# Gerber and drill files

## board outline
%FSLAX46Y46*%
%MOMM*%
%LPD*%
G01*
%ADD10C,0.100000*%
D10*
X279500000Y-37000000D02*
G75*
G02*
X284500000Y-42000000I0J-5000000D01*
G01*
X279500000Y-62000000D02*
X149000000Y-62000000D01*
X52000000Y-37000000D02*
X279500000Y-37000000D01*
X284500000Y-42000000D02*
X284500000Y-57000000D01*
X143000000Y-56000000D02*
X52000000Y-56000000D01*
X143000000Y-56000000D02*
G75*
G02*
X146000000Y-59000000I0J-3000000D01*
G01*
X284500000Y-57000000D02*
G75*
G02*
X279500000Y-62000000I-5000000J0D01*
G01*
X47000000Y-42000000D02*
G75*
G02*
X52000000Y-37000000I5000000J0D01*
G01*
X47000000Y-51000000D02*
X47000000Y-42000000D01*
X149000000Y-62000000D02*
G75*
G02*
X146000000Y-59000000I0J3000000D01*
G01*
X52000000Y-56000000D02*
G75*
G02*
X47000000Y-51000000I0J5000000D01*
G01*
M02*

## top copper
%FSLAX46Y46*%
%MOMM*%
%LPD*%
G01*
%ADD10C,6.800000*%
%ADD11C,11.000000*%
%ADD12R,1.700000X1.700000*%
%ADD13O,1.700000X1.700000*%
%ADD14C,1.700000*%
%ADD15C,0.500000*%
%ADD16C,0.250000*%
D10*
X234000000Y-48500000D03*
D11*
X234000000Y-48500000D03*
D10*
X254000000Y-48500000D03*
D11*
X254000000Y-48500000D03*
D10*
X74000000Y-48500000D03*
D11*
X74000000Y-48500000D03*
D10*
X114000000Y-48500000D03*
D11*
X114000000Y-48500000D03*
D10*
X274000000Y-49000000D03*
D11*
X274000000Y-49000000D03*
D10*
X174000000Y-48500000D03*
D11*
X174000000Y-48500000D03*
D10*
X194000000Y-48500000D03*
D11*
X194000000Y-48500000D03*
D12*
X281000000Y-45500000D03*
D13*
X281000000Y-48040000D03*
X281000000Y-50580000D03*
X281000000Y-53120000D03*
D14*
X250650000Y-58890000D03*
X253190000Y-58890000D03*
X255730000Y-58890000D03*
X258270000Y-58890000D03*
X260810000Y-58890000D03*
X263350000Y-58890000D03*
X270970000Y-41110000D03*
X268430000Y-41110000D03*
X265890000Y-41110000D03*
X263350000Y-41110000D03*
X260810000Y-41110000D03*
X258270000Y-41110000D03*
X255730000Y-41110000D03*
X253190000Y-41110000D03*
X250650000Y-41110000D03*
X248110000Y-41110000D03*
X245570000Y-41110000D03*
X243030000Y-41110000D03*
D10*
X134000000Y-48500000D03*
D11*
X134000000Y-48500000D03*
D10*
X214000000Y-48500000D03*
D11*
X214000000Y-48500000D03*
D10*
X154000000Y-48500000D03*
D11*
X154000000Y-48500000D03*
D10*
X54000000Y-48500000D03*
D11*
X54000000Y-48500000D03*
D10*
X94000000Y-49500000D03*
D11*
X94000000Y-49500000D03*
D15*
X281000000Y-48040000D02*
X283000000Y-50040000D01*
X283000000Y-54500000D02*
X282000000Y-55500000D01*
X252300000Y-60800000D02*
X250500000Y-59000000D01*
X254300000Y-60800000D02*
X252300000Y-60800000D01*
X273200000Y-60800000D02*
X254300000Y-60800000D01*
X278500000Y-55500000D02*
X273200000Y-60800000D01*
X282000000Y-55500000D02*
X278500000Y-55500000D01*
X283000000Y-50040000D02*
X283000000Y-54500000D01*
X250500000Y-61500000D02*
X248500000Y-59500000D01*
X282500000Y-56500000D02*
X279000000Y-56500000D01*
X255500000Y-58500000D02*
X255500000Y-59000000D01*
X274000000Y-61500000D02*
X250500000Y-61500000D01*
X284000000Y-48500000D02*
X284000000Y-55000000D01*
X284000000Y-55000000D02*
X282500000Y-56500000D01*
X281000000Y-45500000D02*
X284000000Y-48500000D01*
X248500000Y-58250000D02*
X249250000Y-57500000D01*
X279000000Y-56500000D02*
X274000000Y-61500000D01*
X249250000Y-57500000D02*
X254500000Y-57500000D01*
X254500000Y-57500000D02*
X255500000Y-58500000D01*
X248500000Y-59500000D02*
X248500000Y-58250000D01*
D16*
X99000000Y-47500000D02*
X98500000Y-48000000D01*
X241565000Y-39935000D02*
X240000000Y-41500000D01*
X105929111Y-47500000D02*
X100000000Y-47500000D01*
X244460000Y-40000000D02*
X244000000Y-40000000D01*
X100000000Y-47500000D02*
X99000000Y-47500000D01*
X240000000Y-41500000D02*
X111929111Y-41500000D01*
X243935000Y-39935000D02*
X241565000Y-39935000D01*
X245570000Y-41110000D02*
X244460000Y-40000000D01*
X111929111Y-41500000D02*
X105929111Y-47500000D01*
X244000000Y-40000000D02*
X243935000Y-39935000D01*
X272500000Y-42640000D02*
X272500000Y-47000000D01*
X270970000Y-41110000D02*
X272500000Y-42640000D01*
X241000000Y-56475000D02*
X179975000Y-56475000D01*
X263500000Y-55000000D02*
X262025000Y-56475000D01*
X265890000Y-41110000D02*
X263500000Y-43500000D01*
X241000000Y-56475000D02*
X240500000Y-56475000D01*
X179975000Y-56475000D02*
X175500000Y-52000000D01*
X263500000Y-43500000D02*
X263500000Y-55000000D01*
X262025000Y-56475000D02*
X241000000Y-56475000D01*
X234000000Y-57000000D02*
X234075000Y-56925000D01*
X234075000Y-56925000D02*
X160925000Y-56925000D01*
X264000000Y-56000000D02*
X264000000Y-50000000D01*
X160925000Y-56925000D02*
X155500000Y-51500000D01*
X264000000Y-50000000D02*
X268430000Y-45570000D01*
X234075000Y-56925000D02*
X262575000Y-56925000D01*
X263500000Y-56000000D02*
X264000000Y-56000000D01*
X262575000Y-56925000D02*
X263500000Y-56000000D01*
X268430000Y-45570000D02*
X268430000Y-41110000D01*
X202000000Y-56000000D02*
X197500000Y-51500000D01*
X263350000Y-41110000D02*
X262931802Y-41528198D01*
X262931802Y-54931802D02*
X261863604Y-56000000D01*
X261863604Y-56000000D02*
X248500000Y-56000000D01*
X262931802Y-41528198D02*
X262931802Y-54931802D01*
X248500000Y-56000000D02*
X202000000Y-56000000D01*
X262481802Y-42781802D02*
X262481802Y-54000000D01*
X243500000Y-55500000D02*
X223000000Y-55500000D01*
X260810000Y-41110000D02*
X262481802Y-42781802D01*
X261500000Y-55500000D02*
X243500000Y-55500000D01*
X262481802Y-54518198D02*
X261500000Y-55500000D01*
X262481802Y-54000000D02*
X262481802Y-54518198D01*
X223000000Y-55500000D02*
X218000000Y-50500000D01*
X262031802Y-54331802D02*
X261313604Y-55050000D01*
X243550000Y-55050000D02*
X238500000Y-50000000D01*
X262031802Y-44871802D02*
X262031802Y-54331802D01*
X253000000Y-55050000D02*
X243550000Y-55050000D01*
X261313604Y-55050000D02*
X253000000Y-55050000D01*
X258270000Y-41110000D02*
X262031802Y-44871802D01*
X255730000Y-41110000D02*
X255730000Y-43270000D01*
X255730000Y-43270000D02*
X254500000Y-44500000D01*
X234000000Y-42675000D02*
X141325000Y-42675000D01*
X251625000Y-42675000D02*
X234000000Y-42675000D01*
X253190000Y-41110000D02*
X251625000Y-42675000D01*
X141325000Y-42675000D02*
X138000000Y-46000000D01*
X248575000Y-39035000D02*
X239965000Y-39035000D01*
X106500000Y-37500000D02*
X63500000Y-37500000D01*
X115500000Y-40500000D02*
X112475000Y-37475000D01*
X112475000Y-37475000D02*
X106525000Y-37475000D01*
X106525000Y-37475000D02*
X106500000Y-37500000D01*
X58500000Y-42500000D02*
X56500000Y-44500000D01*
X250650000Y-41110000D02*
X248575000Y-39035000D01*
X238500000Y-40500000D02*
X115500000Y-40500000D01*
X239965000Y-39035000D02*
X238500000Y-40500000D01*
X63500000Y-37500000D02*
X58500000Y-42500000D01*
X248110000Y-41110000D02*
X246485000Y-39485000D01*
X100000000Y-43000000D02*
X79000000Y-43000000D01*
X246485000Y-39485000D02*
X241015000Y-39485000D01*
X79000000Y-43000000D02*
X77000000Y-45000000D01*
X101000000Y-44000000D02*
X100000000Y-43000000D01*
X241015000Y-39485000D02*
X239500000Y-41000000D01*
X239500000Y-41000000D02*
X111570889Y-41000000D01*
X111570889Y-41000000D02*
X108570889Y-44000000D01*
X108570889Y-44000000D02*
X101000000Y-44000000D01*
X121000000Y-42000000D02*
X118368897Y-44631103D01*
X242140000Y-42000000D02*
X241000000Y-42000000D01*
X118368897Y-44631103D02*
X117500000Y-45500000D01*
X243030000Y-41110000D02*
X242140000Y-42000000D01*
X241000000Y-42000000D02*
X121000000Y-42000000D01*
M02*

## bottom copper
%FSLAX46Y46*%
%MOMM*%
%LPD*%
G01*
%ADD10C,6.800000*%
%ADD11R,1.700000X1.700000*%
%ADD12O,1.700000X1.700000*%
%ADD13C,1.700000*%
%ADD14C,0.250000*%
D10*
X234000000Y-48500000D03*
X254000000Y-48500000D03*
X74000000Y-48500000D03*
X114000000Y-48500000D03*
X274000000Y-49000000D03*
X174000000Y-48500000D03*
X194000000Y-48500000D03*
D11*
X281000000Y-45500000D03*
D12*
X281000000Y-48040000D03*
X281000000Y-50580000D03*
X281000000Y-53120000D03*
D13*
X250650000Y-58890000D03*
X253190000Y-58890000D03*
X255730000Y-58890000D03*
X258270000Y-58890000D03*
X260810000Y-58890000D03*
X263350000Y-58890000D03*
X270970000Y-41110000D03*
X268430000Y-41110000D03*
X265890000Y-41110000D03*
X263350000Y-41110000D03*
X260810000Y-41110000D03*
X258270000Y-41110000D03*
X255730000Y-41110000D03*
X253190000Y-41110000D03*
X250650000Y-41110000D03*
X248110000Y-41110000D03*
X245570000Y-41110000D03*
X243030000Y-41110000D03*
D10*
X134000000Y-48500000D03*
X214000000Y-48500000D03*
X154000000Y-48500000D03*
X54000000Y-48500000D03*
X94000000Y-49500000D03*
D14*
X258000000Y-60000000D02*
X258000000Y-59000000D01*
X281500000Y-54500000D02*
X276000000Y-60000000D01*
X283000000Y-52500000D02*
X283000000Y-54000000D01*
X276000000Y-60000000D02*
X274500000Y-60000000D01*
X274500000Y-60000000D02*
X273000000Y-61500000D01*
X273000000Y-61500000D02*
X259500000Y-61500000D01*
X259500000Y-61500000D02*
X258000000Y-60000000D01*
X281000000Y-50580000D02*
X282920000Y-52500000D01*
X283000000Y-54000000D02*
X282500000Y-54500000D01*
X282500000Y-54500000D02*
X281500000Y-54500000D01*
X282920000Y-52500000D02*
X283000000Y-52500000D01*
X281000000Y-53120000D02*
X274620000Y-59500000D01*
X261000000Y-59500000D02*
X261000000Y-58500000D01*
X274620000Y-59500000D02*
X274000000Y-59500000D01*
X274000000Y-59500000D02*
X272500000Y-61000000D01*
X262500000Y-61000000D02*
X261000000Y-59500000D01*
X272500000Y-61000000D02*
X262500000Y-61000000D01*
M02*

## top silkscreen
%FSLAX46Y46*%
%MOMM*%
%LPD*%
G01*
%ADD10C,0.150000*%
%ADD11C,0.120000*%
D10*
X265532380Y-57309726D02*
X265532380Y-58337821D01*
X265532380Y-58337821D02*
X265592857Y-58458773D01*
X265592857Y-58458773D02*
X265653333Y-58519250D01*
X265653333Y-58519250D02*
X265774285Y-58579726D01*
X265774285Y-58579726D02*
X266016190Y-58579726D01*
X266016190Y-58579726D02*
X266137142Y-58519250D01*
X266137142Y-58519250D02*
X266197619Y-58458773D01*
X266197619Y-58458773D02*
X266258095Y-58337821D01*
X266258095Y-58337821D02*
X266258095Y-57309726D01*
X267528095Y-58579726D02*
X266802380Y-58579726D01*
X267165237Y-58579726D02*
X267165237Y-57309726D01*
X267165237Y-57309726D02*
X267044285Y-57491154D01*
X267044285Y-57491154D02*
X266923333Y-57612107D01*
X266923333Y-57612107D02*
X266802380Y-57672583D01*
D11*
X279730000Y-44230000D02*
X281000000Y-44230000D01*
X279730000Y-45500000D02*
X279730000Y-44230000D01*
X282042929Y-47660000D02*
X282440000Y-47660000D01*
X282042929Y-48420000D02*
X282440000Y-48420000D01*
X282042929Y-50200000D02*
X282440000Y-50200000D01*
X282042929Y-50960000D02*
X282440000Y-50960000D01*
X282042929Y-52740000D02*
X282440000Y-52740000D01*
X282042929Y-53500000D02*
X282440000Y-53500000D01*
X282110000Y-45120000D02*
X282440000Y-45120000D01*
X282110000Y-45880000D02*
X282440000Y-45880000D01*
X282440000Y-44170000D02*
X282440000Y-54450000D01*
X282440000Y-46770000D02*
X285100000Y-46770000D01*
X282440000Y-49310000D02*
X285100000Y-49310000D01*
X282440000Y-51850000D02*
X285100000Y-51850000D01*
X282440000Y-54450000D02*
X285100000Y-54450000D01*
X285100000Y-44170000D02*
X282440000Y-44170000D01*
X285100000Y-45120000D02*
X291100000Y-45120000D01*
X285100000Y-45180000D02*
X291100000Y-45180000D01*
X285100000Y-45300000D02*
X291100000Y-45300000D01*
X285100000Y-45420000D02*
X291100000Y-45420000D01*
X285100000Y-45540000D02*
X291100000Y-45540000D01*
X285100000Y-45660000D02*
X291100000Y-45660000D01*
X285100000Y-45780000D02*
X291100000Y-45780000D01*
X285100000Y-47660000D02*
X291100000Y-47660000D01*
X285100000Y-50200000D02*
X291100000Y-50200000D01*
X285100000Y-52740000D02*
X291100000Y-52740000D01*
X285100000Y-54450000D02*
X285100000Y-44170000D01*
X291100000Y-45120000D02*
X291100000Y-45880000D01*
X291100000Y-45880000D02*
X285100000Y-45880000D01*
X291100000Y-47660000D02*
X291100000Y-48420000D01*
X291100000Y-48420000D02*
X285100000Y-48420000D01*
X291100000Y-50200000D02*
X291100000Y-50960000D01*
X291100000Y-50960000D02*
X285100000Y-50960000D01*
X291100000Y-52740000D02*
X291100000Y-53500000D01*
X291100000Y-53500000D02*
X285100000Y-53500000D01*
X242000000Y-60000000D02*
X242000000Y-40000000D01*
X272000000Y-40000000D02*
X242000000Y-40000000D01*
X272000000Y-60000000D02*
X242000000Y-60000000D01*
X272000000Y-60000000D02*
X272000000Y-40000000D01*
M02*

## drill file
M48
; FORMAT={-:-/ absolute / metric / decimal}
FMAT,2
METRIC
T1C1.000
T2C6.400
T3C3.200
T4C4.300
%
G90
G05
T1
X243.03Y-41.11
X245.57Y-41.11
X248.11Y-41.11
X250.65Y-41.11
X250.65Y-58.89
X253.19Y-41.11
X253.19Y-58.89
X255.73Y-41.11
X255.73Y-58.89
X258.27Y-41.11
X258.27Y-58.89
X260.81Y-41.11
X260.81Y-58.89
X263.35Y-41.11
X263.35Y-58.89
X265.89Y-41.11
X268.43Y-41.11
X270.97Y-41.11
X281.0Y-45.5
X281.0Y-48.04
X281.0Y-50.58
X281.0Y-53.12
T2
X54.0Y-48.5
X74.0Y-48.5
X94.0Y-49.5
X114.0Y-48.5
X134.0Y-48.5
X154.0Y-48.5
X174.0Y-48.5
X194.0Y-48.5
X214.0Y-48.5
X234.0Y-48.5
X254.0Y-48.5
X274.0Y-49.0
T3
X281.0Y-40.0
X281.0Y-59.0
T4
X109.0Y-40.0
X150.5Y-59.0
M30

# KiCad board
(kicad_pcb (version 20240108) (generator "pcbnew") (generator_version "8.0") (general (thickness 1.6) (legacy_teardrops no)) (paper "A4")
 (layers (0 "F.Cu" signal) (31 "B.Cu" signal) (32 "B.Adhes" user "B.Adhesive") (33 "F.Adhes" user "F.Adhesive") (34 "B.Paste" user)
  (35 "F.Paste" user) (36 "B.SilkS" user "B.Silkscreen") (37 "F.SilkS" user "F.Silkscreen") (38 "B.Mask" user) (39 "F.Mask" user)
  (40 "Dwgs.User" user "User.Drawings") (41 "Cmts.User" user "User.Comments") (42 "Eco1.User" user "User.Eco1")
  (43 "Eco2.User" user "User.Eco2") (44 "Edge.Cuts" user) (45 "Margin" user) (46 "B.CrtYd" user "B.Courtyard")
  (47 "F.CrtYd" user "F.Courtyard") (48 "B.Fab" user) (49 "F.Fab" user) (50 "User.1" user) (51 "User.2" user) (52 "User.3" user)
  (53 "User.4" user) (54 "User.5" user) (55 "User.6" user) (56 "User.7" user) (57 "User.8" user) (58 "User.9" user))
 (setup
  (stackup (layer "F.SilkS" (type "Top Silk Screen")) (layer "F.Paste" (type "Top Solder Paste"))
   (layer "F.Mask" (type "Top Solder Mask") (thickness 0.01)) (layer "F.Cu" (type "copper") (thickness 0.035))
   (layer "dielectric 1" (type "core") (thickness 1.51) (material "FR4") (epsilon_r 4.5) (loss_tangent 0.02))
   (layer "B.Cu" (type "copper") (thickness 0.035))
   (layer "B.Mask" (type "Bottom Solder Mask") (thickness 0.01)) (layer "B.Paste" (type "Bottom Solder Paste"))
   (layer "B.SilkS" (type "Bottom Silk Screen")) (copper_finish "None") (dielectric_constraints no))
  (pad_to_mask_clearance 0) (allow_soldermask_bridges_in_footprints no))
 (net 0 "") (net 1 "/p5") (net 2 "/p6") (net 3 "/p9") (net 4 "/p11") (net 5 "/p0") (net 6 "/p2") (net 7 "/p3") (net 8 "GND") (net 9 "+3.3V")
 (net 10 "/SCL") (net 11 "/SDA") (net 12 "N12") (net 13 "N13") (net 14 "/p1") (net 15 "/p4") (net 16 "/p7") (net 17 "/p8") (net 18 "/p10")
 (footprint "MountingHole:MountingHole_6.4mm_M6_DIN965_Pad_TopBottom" (layer "F.Cu") (at 234 48.5 90)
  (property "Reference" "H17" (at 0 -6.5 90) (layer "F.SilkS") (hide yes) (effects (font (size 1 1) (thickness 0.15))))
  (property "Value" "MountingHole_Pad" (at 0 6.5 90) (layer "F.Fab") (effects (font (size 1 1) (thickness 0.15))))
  (pad "" connect circle (at 0 0 90) (size 11 11) (layers "B.Mask" "Rescue"))
  (pad "1" thru_hole circle (at 0 0 90) (size 6.8 6.8) (drill 6.4) (layers "*.Cu" "*.Mask") (remove_unused_layers no) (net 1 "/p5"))
  (pad "1" connect circle (at 0 0 90) (size 11 11) (layers "F.Cu" "F.Mask") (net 1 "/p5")))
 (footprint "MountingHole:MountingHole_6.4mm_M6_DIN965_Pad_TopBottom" (layer "F.Cu") (at 254 48.5 90)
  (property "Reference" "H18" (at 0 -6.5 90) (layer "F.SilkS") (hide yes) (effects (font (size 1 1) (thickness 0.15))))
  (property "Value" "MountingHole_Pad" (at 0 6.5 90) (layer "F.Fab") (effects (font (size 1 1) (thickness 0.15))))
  (pad "" connect circle (at 0 0 90) (size 11 11) (layers "B.Mask" "Rescue"))
  (pad "1" thru_hole circle (at 0 0 90) (size 6.8 6.8) (drill 6.4) (layers "*.Cu" "*.Mask") (remove_unused_layers no) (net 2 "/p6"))
  (pad "1" connect circle (at 0 0 90) (size 11 11) (layers "F.Cu" "F.Mask") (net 2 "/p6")))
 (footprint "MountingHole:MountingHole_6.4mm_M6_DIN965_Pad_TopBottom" (layer "F.Cu") (at 74 48.5)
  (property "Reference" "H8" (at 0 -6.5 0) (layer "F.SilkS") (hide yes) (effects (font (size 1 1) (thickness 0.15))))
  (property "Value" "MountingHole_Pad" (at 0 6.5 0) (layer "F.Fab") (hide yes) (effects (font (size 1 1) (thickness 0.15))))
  (pad "" connect circle (at 0 0) (size 11 11) (layers "B.Mask" "Rescue"))
  (pad "1" thru_hole circle (at 0 0) (size 6.8 6.8) (drill 6.4) (layers "*.Cu" "*.Mask") (remove_unused_layers no) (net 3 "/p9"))
  (pad "1" connect circle (at 0 0) (size 11 11) (layers "F.Cu" "F.Mask") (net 3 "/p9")))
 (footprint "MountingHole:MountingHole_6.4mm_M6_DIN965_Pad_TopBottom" (layer "F.Cu") (at 114 48.5 90)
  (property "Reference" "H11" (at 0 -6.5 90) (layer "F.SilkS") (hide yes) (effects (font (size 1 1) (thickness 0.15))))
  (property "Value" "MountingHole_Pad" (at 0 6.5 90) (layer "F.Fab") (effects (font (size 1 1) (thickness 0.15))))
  (pad "" connect circle (at 0 0 90) (size 11 11) (layers "B.Mask" "Rescue"))
  (pad "1" thru_hole circle (at 0 0 90) (size 6.8 6.8) (drill 6.4) (layers "*.Cu" "*.Mask") (remove_unused_layers no) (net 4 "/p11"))
  (pad "1" connect circle (at 0 0 90) (size 11 11) (layers "F.Cu" "F.Mask") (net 4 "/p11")))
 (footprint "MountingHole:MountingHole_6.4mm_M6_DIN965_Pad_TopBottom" (layer "F.Cu") (at 274 49 90)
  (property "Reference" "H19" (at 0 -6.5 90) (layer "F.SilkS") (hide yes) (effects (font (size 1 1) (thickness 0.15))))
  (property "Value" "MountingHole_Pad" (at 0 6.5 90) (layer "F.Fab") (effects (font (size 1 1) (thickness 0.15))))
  (pad "" connect circle (at 0 0 90) (size 11 11) (layers "B.Mask" "Rescue"))
  (pad "1" thru_hole circle (at 0 0 90) (size 6.8 6.8) (drill 6.4) (layers "*.Cu" "*.Mask") (remove_unused_layers no) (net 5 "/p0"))
  (pad "1" connect circle (at 0 0 90) (size 11 11) (layers "F.Cu" "F.Mask") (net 5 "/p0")))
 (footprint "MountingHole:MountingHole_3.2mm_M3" (layer "F.Cu") (at 283.7475 40.08 -90)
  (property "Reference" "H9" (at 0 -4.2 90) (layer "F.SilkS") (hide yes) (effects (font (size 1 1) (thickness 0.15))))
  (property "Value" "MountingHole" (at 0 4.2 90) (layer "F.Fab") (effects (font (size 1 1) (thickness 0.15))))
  (pad "" np_thru_hole circle (at -0.08 2.7475 270) (size 3.2 3.2) (drill 3.2) (layers "F&B.Cu" "*.Mask")))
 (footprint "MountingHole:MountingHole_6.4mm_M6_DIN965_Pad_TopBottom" (layer "F.Cu") (at 174 48.5 90)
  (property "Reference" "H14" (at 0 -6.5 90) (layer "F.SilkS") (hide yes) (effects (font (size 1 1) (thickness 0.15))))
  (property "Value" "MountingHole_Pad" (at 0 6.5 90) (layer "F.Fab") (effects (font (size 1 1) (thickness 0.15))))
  (pad "" connect circle (at 0 0 90) (size 11 11) (layers "B.Mask" "Rescue"))
  (pad "1" thru_hole circle (at 0 0 90) (size 6.8 6.8) (drill 6.4) (layers "*.Cu" "*.Mask") (remove_unused_layers no) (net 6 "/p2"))
  (pad "1" connect circle (at 0 0 90) (size 11 11) (layers "F.Cu" "F.Mask") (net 6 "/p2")))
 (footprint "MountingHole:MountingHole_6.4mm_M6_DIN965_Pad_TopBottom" (layer "F.Cu") (at 194 48.5 90)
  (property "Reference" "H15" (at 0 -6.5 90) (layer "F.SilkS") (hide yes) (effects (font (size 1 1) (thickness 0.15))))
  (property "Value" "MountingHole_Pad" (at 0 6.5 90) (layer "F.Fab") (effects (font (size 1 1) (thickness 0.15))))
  (pad "" connect circle (at 0 0 90) (size 11 11) (layers "B.Mask" "Rescue"))
  (pad "1" thru_hole circle (at 0 0 90) (size 6.8 6.8) (drill 6.4) (layers "*.Cu" "*.Mask") (remove_unused_layers no) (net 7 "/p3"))
  (pad "1" connect circle (at 0 0 90) (size 11 11) (layers "F.Cu" "F.Mask") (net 7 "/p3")))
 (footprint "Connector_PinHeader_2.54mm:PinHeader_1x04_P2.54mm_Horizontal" (layer "F.Cu") (at 281 45.5)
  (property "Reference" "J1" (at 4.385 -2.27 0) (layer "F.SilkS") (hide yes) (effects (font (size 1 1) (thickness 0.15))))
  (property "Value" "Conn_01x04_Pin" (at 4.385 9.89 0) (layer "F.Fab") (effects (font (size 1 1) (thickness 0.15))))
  (fp_line (start -1.27 -1.27) (end 0 -1.27) (stroke (width 0.12) (type solid)) (layer "F.SilkS"))
  (fp_line (start -1.27 0) (end -1.27 -1.27) (stroke (width 0.12) (type solid)) (layer "F.SilkS"))
  (fp_line (start 1.042929 2.16) (end 1.44 2.16) (stroke (width 0.12) (type solid)) (layer "F.SilkS"))
  (fp_line (start 1.042929 2.92) (end 1.44 2.92) (stroke (width 0.12) (type solid)) (layer "F.SilkS"))
  (fp_line (start 1.042929 4.7) (end 1.44 4.7) (stroke (width 0.12) (type solid)) (layer "F.SilkS"))
  (fp_line (start 1.042929 5.46) (end 1.44 5.46) (stroke (width 0.12) (type solid)) (layer "F.SilkS"))
  (fp_line (start 1.042929 7.24) (end 1.44 7.24) (stroke (width 0.12) (type solid)) (layer "F.SilkS"))
  (fp_line (start 1.042929 8) (end 1.44 8) (stroke (width 0.12) (type solid)) (layer "F.SilkS"))
  (fp_line (start 1.11 -0.38) (end 1.44 -0.38) (stroke (width 0.12) (type solid)) (layer "F.SilkS"))
  (fp_line (start 1.11 0.38) (end 1.44 0.38) (stroke (width 0.12) (type solid)) (layer "F.SilkS"))
  (fp_line (start 1.44 -1.33) (end 1.44 8.95) (stroke (width 0.12) (type solid)) (layer "F.SilkS"))
  (fp_line (start 1.44 1.27) (end 4.1 1.27) (stroke (width 0.12) (type solid)) (layer "F.SilkS"))
  (fp_line (start 1.44 3.81) (end 4.1 3.81) (stroke (width 0.12) (type solid)) (layer "F.SilkS"))
  (fp_line (start 1.44 6.35) (end 4.1 6.35) (stroke (width 0.12) (type solid)) (layer "F.SilkS"))
  (fp_line (start 1.44 8.95) (end 4.1 8.95) (stroke (width 0.12) (type solid)) (layer "F.SilkS"))
  (fp_line (start 4.1 -1.33) (end 1.44 -1.33) (stroke (width 0.12) (type solid)) (layer "F.SilkS"))
  (fp_line (start 4.1 -0.38) (end 10.1 -0.38) (stroke (width 0.12) (type solid)) (layer "F.SilkS"))
  (fp_line (start 4.1 -0.32) (end 10.1 -0.32) (stroke (width 0.12) (type solid)) (layer "F.SilkS"))
  (fp_line (start 4.1 -0.2) (end 10.1 -0.2) (stroke (width 0.12) (type solid)) (layer "F.SilkS"))
  (fp_line (start 4.1 -0.08) (end 10.1 -0.08) (stroke (width 0.12) (type solid)) (layer "F.SilkS"))
  (fp_line (start 4.1 0.04) (end 10.1 0.04) (stroke (width 0.12) (type solid)) (layer "F.SilkS"))
  (fp_line (start 4.1 0.16) (end 10.1 0.16) (stroke (width 0.12) (type solid)) (layer "F.SilkS"))
  (fp_line (start 4.1 0.28) (end 10.1 0.28) (stroke (width 0.12) (type solid)) (layer "F.SilkS"))
  (fp_line (start 4.1 2.16) (end 10.1 2.16) (stroke (width 0.12) (type solid)) (layer "F.SilkS"))
  (fp_line (start 4.1 4.7) (end 10.1 4.7) (stroke (width 0.12) (type solid)) (layer "F.SilkS"))
  (fp_line (start 4.1 7.24) (end 10.1 7.24) (stroke (width 0.12) (type solid)) (layer "F.SilkS"))
  (fp_line (start 4.1 8.95) (end 4.1 -1.33) (stroke (width 0.12) (type solid)) (layer "F.SilkS"))
  (fp_line (start 10.1 -0.38) (end 10.1 0.38) (stroke (width 0.12) (type solid)) (layer "F.SilkS"))
  (fp_line (start 10.1 0.38) (end 4.1 0.38) (stroke (width 0.12) (type solid)) (layer "F.SilkS"))
  (fp_line (start 10.1 2.16) (end 10.1 2.92) (stroke (width 0.12) (type solid)) (layer "F.SilkS"))
  (fp_line (start 10.1 2.92) (end 4.1 2.92) (stroke (width 0.12) (type solid)) (layer "F.SilkS"))
  (fp_line (start 10.1 4.7) (end 10.1 5.46) (stroke (width 0.12) (type solid)) (layer "F.SilkS"))
  (fp_line (start 10.1 5.46) (end 4.1 5.46) (stroke (width 0.12) (type solid)) (layer "F.SilkS"))
  (fp_line (start 10.1 7.24) (end 10.1 8) (stroke (width 0.12) (type solid)) (layer "F.SilkS"))
  (fp_line (start 10.1 8) (end 4.1 8) (stroke (width 0.12) (type solid)) (layer "F.SilkS"))
  (pad "1" thru_hole rect (at 0 0) (size 1.7 1.7) (drill 1) (layers "*.Cu" "*.Mask") (remove_unused_layers no) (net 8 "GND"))
  (pad "2" thru_hole oval (at 0 2.54) (size 1.7 1.7) (drill 1) (layers "*.Cu" "*.Mask") (remove_unused_layers no) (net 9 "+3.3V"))
  (pad "3" thru_hole oval (at 0 5.08) (size 1.7 1.7) (drill 1) (layers "*.Cu" "*.Mask") (remove_unused_layers no) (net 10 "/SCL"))
  (pad "4" thru_hole oval (at 0 7.62) (size 1.7 1.7) (drill 1) (layers "*.Cu" "*.Mask") (remove_unused_layers no) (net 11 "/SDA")))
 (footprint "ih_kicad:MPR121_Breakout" (layer "F.Cu") (at 257 50 180)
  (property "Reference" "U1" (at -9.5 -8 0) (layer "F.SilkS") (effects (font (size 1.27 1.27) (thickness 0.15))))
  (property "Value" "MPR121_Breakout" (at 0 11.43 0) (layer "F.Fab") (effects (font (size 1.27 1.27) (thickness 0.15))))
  (fp_line (start 15 -10) (end 15 10) (stroke (width 0.12) (type solid)) (layer "F.SilkS"))
  (fp_line (start -15 10) (end 15 10) (stroke (width 0.12) (type solid)) (layer "F.SilkS"))
  (fp_line (start -15 -10) (end 15 -10) (stroke (width 0.12) (type solid)) (layer "F.SilkS"))
  (fp_line (start -15 -10) (end -15 10) (stroke (width 0.12) (type solid)) (layer "F.SilkS"))
  (pad "1" thru_hole circle (at 6.35 -8.89 180) (size 1.7 1.7) (drill 1) (layers "*.Cu" "*.Mask") (remove_unused_layers no) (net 9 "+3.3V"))
  (pad "2" thru_hole circle (at 3.81 -8.89 180) (size 1.7 1.7) (drill 1) (layers "*.Cu" "*.Mask") (remove_unused_layers no) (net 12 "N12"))
  (pad "3" thru_hole circle (at 1.27 -8.89 180) (size 1.7 1.7) (drill 1) (layers "*.Cu" "*.Mask") (remove_unused_layers no) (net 8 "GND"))
  (pad "4" thru_hole circle (at -1.27 -8.89 180) (size 1.7 1.7) (drill 1) (layers "*.Cu" "*.Mask") (remove_unused_layers no) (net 10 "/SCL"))
  (pad "5" thru_hole circle (at -3.81 -8.89 180) (size 1.7 1.7) (drill 1) (layers "*.Cu" "*.Mask") (remove_unused_layers no) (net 11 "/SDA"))
  (pad "6" thru_hole circle (at -6.35 -8.89 180) (size 1.7 1.7) (drill 1) (layers "*.Cu" "*.Mask") (remove_unused_layers no) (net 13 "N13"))
  (pad "7" thru_hole circle (at -13.97 8.89 180) (size 1.7 1.7) (drill 1) (layers "*.Cu" "*.Mask") (remove_unused_layers no) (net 5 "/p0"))
  (pad "8" thru_hole circle (at -11.43 8.89 180) (size 1.7 1.7) (drill 1) (layers "*.Cu" "*.Mask") (remove_unused_layers no) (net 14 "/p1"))
  (pad "9" thru_hole circle (at -8.89 8.89 180) (size 1.7 1.7) (drill 1) (layers "*.Cu" "*.Mask") (remove_unused_layers no) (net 6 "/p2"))
  (pad "10" thru_hole circle (at -6.35 8.89 180) (size 1.7 1.7) (drill 1) (layers "*.Cu" "*.Mask") (remove_unused_layers no) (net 7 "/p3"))
  (pad "11" thru_hole circle (at -3.81 8.89 180) (size 1.7 1.7) (drill 1) (layers "*.Cu" "*.Mask") (remove_unused_layers no) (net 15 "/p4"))
  (pad "12" thru_hole circle (at -1.27 8.89 180) (size 1.7 1.7) (drill 1) (layers "*.Cu" "*.Mask") (remove_unused_layers no) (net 1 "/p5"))
  (pad "13" thru_hole circle (at 1.27 8.89 180) (size 1.7 1.7) (drill 1) (layers "*.Cu" "*.Mask") (remove_unused_layers no) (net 2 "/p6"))
  (pad "14" thru_hole circle (at 3.81 8.89 180) (size 1.7 1.7) (drill 1) (layers "*.Cu" "*.Mask") (remove_unused_layers no) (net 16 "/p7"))
  (pad "15" thru_hole circle (at 6.35 8.89 180) (size 1.7 1.7) (drill 1) (layers "*.Cu" "*.Mask") (remove_unused_layers no) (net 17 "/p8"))
  (pad "16" thru_hole circle (at 8.89 8.89 180) (size 1.7 1.7) (drill 1) (layers "*.Cu" "*.Mask") (remove_unused_layers no) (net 3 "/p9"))
  (pad "17" thru_hole circle (at 11.43 8.89 180) (size 1.7 1.7) (drill 1) (layers "*.Cu" "*.Mask") (remove_unused_layers no) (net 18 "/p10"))
  (pad "18" thru_hole circle (at 13.97 8.89 180) (size 1.7 1.7) (drill 1) (layers "*.Cu" "*.Mask") (remove_unused_layers no) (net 4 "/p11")))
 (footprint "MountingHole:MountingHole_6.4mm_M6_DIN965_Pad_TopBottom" (layer "F.Cu") (at 134 48.5 90)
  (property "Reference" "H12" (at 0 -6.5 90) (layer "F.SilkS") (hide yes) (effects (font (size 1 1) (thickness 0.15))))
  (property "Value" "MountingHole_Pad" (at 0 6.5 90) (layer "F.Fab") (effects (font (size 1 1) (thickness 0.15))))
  (pad "" connect circle (at 0 0 90) (size 11 11) (layers "B.Mask" "Rescue"))
  (pad "1" thru_hole circle (at 0 0 90) (size 6.8 6.8) (drill 6.4) (layers "*.Cu" "*.Mask") (remove_unused_layers no) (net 16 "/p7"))
  (pad "1" connect circle (at 0 0 90) (size 11 11) (layers "F.Cu" "F.Mask") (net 16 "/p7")))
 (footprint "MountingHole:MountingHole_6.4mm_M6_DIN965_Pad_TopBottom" (layer "F.Cu") (at 214 48.5 90)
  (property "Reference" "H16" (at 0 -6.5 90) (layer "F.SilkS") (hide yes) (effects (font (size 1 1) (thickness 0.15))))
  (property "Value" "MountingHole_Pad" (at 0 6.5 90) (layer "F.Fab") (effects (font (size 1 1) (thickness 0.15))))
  (pad "" connect circle (at 0 0 90) (size 11 11) (layers "B.Mask" "Rescue"))
  (pad "1" thru_hole circle (at 0 0 90) (size 6.8 6.8) (drill 6.4) (layers "*.Cu" "*.Mask") (remove_unused_layers no) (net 15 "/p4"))
  (pad "1" connect circle (at 0 0 90) (size 11 11) (layers "F.Cu" "F.Mask") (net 15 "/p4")))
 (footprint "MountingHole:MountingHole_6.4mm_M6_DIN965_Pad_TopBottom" (layer "F.Cu") (at 154 48.5 90)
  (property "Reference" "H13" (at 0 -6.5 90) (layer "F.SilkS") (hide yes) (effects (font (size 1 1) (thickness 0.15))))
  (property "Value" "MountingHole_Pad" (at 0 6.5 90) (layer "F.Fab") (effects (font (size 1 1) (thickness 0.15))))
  (pad "" connect circle (at 0 0 90) (size 11 11) (layers "B.Mask" "Rescue"))
  (pad "1" thru_hole circle (at 0 0 90) (size 6.8 6.8) (drill 6.4) (layers "*.Cu" "*.Mask") (remove_unused_layers no) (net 14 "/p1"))
  (pad "1" connect circle (at 0 0 90) (size 11 11) (layers "F.Cu" "F.Mask") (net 14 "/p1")))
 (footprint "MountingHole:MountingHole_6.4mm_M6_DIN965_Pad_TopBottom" (layer "F.Cu") (at 54 48.5)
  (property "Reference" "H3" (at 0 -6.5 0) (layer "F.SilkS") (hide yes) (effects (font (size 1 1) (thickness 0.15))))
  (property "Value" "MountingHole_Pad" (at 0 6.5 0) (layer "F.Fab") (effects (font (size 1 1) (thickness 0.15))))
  (pad "" connect circle (at 0 0) (size 11 11) (layers "B.Mask" "Rescue"))
  (pad "1" thru_hole circle (at 0 0) (size 6.8 6.8) (drill 6.4) (layers "*.Cu" "*.Mask") (remove_unused_layers no) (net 17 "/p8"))
  (pad "1" connect circle (at 0 0) (size 11 11) (layers "F.Cu" "F.Mask") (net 17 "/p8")))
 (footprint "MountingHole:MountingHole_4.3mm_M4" (layer "F.Cu") (at 118 97.5)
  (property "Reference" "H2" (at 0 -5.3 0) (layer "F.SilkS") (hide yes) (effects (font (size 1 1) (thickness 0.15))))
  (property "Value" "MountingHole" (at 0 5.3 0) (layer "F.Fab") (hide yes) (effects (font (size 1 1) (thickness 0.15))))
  (pad "" np_thru_hole circle (at -9 -57.5) (size 4.3 4.3) (drill 4.3) (layers "F&B.Cu" "*.Mask")))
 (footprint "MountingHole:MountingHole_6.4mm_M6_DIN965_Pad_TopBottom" (layer "F.Cu") (at 94 49.5)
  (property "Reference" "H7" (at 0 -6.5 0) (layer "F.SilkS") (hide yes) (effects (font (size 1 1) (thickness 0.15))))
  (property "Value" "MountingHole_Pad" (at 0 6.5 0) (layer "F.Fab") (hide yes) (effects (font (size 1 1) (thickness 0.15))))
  (pad "" connect circle (at 0 0) (size 11 11) (layers "B.Mask" "Rescue"))
  (pad "1" thru_hole circle (at 0 0) (size 6.8 6.8) (drill 6.4) (layers "*.Cu" "*.Mask") (remove_unused_layers no) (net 18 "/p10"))
  (pad "1" connect circle (at 0 0) (size 11 11) (layers "F.Cu" "F.Mask") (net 18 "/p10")))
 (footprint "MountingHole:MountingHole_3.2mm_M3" (layer "F.Cu") (at 278.7475 74.58 -90)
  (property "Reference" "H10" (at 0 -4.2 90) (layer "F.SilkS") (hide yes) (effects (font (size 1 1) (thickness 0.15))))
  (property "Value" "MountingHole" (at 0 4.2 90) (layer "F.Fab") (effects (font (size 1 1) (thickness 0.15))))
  (pad "" np_thru_hole circle (at -15.58 -2.2525 270) (size 3.2 3.2) (drill 3.2) (layers "F&B.Cu" "*.Mask")))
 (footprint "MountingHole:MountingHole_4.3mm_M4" (layer "F.Cu") (at 146.5 97.5)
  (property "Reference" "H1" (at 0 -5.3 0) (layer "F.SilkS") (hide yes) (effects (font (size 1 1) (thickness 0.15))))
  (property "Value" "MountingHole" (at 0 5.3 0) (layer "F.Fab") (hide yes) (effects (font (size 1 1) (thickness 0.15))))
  (pad "" np_thru_hole circle (at 4 -38.5) (size 4.3 4.3) (drill 4.3) (layers "F&B.Cu" "*.Mask")))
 (gr_arc (start 279.5 37) (mid 283.035534 38.464466) (end 284.5 42) (stroke (width 0.1) (type default)) (layer "Edge.Cuts"))
 (gr_line (start 279.5 62) (end 149 62) (stroke (width 0.1) (type default)) (layer "Edge.Cuts"))
 (gr_line (start 52 37) (end 279.5 37) (stroke (width 0.1) (type default)) (layer "Edge.Cuts"))
 (gr_line (start 284.5 42) (end 284.5 57) (stroke (width 0.1) (type default)) (layer "Edge.Cuts"))
 (gr_line (start 143 56) (end 52 56) (stroke (width 0.1) (type default)) (layer "Edge.Cuts"))
 (gr_arc (start 143 56) (mid 145.12132 56.87868) (end 146 59) (stroke (width 0.1) (type default)) (layer "Edge.Cuts"))
 (gr_arc (start 284.5 57) (mid 283.035534 60.535534) (end 279.5 62) (stroke (width 0.1) (type default)) (layer "Edge.Cuts"))
 (gr_arc (start 47 42) (mid 48.464466 38.464466) (end 52 37) (stroke (width 0.1) (type default)) (layer "Edge.Cuts"))
 (gr_line (start 47 51) (end 47 42) (stroke (width 0.1) (type default)) (layer "Edge.Cuts"))
 (gr_arc (start 149 62) (mid 146.87868 61.12132) (end 146 59) (stroke (width 0.1) (type default)) (layer "Edge.Cuts"))
 (gr_arc (start 52 56) (mid 48.464466 54.535534) (end 47 51) (stroke (width 0.1) (type default)) (layer "Edge.Cuts"))
 (segment (start 281 48.04) (end 283 50.04) (width 0.5) (layer "F.Cu") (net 9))
 (segment (start 283 54.5) (end 282 55.5) (width 0.5) (layer "F.Cu") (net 9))
 (segment (start 252.3 60.8) (end 250.5 59) (width 0.5) (layer "F.Cu") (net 9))
 (segment (start 254.3 60.8) (end 252.3 60.8) (width 0.5) (layer "F.Cu") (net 9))
 (segment (start 273.2 60.8) (end 254.3 60.8) (width 0.5) (layer "F.Cu") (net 9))
 (segment (start 278.5 55.5) (end 273.2 60.8) (width 0.5) (layer "F.Cu") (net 9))
 (segment (start 282 55.5) (end 278.5 55.5) (width 0.5) (layer "F.Cu") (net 9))
 (segment (start 283 50.04) (end 283 54.5) (width 0.5) (layer "F.Cu") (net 9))
 (segment (start 250.5 61.5) (end 248.5 59.5) (width 0.5) (layer "F.Cu") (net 8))
 (segment (start 282.5 56.5) (end 279 56.5) (width 0.5) (layer "F.Cu") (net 8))
 (segment (start 255.5 58.5) (end 255.5 59) (width 0.5) (layer "F.Cu") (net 8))
 (segment (start 274 61.5) (end 250.5 61.5) (width 0.5) (layer "F.Cu") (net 8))
 (segment (start 284 48.5) (end 284 55) (width 0.5) (layer "F.Cu") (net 8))
 (segment (start 284 55) (end 282.5 56.5) (width 0.5) (layer "F.Cu") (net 8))
 (segment (start 281 45.5) (end 284 48.5) (width 0.5) (layer "F.Cu") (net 8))
 (segment (start 248.5 58.25) (end 249.25 57.5) (width 0.5) (layer "F.Cu") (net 8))
 (segment (start 279 56.5) (end 274 61.5) (width 0.5) (layer "F.Cu") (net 8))
 (segment (start 249.25 57.5) (end 254.5 57.5) (width 0.5) (layer "F.Cu") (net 8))
 (segment (start 254.5 57.5) (end 255.5 58.5) (width 0.5) (layer "F.Cu") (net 8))
 (segment (start 248.5 59.5) (end 248.5 58.25) (width 0.5) (layer "F.Cu") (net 8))
 (segment (start 99 47.5) (end 98.5 48) (width 0.25) (layer "F.Cu") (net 18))
 (segment (start 241.565 39.935) (end 240 41.5) (width 0.25) (layer "F.Cu") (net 18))
 (segment (start 105.929111 47.5) (end 100 47.5) (width 0.25) (layer "F.Cu") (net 18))
 (segment (start 244.46 40) (end 244 40) (width 0.25) (layer "F.Cu") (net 18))
 (segment (start 100 47.5) (end 99 47.5) (width 0.25) (layer "F.Cu") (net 18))
 (segment (start 240 41.5) (end 111.929111 41.5) (width 0.25) (layer "F.Cu") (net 18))
 (segment (start 243.935 39.935) (end 241.565 39.935) (width 0.25) (layer "F.Cu") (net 18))
 (segment (start 245.57 41.11) (end 244.46 40) (width 0.25) (layer "F.Cu") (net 18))
 (segment (start 111.929111 41.5) (end 105.929111 47.5) (width 0.25) (layer "F.Cu") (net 18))
 (segment (start 244 40) (end 243.935 39.935) (width 0.25) (layer "F.Cu") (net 18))
 (segment (start 272.5 42.64) (end 272.5 47) (width 0.25) (layer "F.Cu") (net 5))
 (segment (start 270.97 41.11) (end 272.5 42.64) (width 0.25) (layer "F.Cu") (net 5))
 (segment (start 241 56.475) (end 179.975 56.475) (width 0.25) (layer "F.Cu") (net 6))
 (segment (start 263.5 55) (end 262.025 56.475) (width 0.25) (layer "F.Cu") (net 6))
 (segment (start 265.89 41.11) (end 263.5 43.5) (width 0.25) (layer "F.Cu") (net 6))
 (segment (start 241 56.475) (end 240.5 56.475) (width 0.25) (layer "F.Cu") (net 6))
 (segment (start 179.975 56.475) (end 175.5 52) (width 0.25) (layer "F.Cu") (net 6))
 (segment (start 263.5 43.5) (end 263.5 55) (width 0.25) (layer "F.Cu") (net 6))
 (segment (start 262.025 56.475) (end 241 56.475) (width 0.25) (layer "F.Cu") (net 6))
 (segment (start 258 60) (end 258 59) (width 0.25) (layer "B.Cu") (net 10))
 (segment (start 281.5 54.5) (end 276 60) (width 0.25) (layer "B.Cu") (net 10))
 (segment (start 283 52.5) (end 283 54) (width 0.25) (layer "B.Cu") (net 10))
 (segment (start 276 60) (end 274.5 60) (width 0.25) (layer "B.Cu") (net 10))
 (segment (start 274.5 60) (end 273 61.5) (width 0.25) (layer "B.Cu") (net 10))
 (segment (start 273 61.5) (end 259.5 61.5) (width 0.25) (layer "B.Cu") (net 10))
 (segment (start 259.5 61.5) (end 258 60) (width 0.25) (layer "B.Cu") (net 10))
 (segment (start 281 50.58) (end 282.92 52.5) (width 0.25) (layer "B.Cu") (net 10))
 (segment (start 283 54) (end 282.5 54.5) (width 0.25) (layer "B.Cu") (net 10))
 (segment (start 282.5 54.5) (end 281.5 54.5) (width 0.25) (layer "B.Cu") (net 10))
 (segment (start 282.92 52.5) (end 283 52.5) (width 0.25) (layer "B.Cu") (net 10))
 (segment (start 281 53.12) (end 274.62 59.5) (width 0.25) (layer "B.Cu") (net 11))
 (segment (start 261 59.5) (end 261 58.5) (width 0.25) (layer "B.Cu") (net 11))
 (segment (start 274.62 59.5) (end 274 59.5) (width 0.25) (layer "B.Cu") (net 11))
 (segment (start 274 59.5) (end 272.5 61) (width 0.25) (layer "B.Cu") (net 11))
 (segment (start 262.5 61) (end 261 59.5) (width 0.25) (layer "B.Cu") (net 11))
 (segment (start 272.5 61) (end 262.5 61) (width 0.25) (layer "B.Cu") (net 11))
 (segment (start 234 57) (end 234.075 56.925) (width 0.25) (layer "F.Cu") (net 14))
 (segment (start 234.075 56.925) (end 160.925 56.925) (width 0.25) (layer "F.Cu") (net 14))
 (segment (start 264 56) (end 264 50) (width 0.25) (layer "F.Cu") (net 14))
 (segment (start 160.925 56.925) (end 155.5 51.5) (width 0.25) (layer "F.Cu") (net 14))
 (segment (start 264 50) (end 268.43 45.57) (width 0.25) (layer "F.Cu") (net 14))
 (segment (start 234.075 56.925) (end 262.575 56.925) (width 0.25) (layer "F.Cu") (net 14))
 (segment (start 263.5 56) (end 264 56) (width 0.25) (layer "F.Cu") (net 14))
 (segment (start 262.575 56.925) (end 263.5 56) (width 0.25) (layer "F.Cu") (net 14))
 (segment (start 268.43 45.57) (end 268.43 41.11) (width 0.25) (layer "F.Cu") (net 14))
 (segment (start 202 56) (end 197.5 51.5) (width 0.25) (layer "F.Cu") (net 7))
 (segment (start 263.35 41.11) (end 262.931802 41.528198) (width 0.25) (layer "F.Cu") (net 7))
 (segment (start 262.931802 54.931802) (end 261.863604 56) (width 0.25) (layer "F.Cu") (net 7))
 (segment (start 261.863604 56) (end 248.5 56) (width 0.25) (layer "F.Cu") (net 7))
 (segment (start 262.931802 41.528198) (end 262.931802 54.931802) (width 0.25) (layer "F.Cu") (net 7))
 (segment (start 248.5 56) (end 202 56) (width 0.25) (layer "F.Cu") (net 7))
 (segment (start 262.481802 42.781802) (end 262.481802 54) (width 0.25) (layer "F.Cu") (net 15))
 (segment (start 243.5 55.5) (end 223 55.5) (width 0.25) (layer "F.Cu") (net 15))
 (segment (start 260.81 41.11) (end 262.481802 42.781802) (width 0.25) (layer "F.Cu") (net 15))
 (segment (start 261.5 55.5) (end 243.5 55.5) (width 0.25) (layer "F.Cu") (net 15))
 (segment (start 262.481802 54.518198) (end 261.5 55.5) (width 0.25) (layer "F.Cu") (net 15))
 (segment (start 262.481802 54) (end 262.481802 54.518198) (width 0.25) (layer "F.Cu") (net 15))
 (segment (start 223 55.5) (end 218 50.5) (width 0.25) (layer "F.Cu") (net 15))
 (segment (start 262.031802 54.331802) (end 261.313604 55.05) (width 0.25) (layer "F.Cu") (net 1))
 (segment (start 243.55 55.05) (end 238.5 50) (width 0.25) (layer "F.Cu") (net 1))
 (segment (start 262.031802 44.871802) (end 262.031802 54.331802) (width 0.25) (layer "F.Cu") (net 1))
 (segment (start 253 55.05) (end 243.55 55.05) (width 0.25) (layer "F.Cu") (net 1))
 (segment (start 261.313604 55.05) (end 253 55.05) (width 0.25) (layer "F.Cu") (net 1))
 (segment (start 258.27 41.11) (end 262.031802 44.871802) (width 0.25) (layer "F.Cu") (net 1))
 (segment (start 255.73 41.11) (end 255.73 43.27) (width 0.25) (layer "F.Cu") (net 2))
 (segment (start 255.73 43.27) (end 254.5 44.5) (width 0.25) (layer "F.Cu") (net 2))
 (segment (start 234 42.675) (end 141.325 42.675) (width 0.25) (layer "F.Cu") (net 16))
 (segment (start 251.625 42.675) (end 234 42.675) (width 0.25) (layer "F.Cu") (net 16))
 (segment (start 253.19 41.11) (end 251.625 42.675) (width 0.25) (layer "F.Cu") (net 16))
 (segment (start 141.325 42.675) (end 138 46) (width 0.25) (layer "F.Cu") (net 16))
 (segment (start 248.575 39.035) (end 239.965 39.035) (width 0.25) (layer "F.Cu") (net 17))
 (segment (start 106.5 37.5) (end 63.5 37.5) (width 0.25) (layer "F.Cu") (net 17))
 (segment (start 115.5 40.5) (end 112.475 37.475) (width 0.25) (layer "F.Cu") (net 17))
 (segment (start 112.475 37.475) (end 106.525 37.475) (width 0.25) (layer "F.Cu") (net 17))
 (segment (start 106.525 37.475) (end 106.5 37.5) (width 0.25) (layer "F.Cu") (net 17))
 (segment (start 58.5 42.5) (end 56.5 44.5) (width 0.25) (layer "F.Cu") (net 17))
 (segment (start 250.65 41.11) (end 248.575 39.035) (width 0.25) (layer "F.Cu") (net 17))
 (segment (start 238.5 40.5) (end 115.5 40.5) (width 0.25) (layer "F.Cu") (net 17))
 (segment (start 239.965 39.035) (end 238.5 40.5) (width 0.25) (layer "F.Cu") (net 17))
 (segment (start 63.5 37.5) (end 58.5 42.5) (width 0.25) (layer "F.Cu") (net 17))
 (segment (start 248.11 41.11) (end 246.485 39.485) (width 0.25) (layer "F.Cu") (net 3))
 (segment (start 100 43) (end 79 43) (width 0.25) (layer "F.Cu") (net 3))
 (segment (start 246.485 39.485) (end 241.015 39.485) (width 0.25) (layer "F.Cu") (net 3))
 (segment (start 79 43) (end 77 45) (width 0.25) (layer "F.Cu") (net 3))
 (segment (start 101 44) (end 100 43) (width 0.25) (layer "F.Cu") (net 3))
 (segment (start 241.015 39.485) (end 239.5 41) (width 0.25) (layer "F.Cu") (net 3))
 (segment (start 239.5 41) (end 111.570889 41) (width 0.25) (layer "F.Cu") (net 3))
 (segment (start 111.570889 41) (end 108.570889 44) (width 0.25) (layer "F.Cu") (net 3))
 (segment (start 108.570889 44) (end 101 44) (width 0.25) (layer "F.Cu") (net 3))
 (segment (start 121 42) (end 118.368897 44.631103) (width 0.25) (layer "F.Cu") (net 4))
 (segment (start 242.14 42) (end 241 42) (width 0.25) (layer "F.Cu") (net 4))
 (segment (start 118.368897 44.631103) (end 117.5 45.5) (width 0.25) (layer "F.Cu") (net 4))
 (segment (start 243.03 41.11) (end 242.14 42) (width 0.25) (layer "F.Cu") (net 4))
 (segment (start 241 42) (end 121 42) (width 0.25) (layer "F.Cu") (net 4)))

